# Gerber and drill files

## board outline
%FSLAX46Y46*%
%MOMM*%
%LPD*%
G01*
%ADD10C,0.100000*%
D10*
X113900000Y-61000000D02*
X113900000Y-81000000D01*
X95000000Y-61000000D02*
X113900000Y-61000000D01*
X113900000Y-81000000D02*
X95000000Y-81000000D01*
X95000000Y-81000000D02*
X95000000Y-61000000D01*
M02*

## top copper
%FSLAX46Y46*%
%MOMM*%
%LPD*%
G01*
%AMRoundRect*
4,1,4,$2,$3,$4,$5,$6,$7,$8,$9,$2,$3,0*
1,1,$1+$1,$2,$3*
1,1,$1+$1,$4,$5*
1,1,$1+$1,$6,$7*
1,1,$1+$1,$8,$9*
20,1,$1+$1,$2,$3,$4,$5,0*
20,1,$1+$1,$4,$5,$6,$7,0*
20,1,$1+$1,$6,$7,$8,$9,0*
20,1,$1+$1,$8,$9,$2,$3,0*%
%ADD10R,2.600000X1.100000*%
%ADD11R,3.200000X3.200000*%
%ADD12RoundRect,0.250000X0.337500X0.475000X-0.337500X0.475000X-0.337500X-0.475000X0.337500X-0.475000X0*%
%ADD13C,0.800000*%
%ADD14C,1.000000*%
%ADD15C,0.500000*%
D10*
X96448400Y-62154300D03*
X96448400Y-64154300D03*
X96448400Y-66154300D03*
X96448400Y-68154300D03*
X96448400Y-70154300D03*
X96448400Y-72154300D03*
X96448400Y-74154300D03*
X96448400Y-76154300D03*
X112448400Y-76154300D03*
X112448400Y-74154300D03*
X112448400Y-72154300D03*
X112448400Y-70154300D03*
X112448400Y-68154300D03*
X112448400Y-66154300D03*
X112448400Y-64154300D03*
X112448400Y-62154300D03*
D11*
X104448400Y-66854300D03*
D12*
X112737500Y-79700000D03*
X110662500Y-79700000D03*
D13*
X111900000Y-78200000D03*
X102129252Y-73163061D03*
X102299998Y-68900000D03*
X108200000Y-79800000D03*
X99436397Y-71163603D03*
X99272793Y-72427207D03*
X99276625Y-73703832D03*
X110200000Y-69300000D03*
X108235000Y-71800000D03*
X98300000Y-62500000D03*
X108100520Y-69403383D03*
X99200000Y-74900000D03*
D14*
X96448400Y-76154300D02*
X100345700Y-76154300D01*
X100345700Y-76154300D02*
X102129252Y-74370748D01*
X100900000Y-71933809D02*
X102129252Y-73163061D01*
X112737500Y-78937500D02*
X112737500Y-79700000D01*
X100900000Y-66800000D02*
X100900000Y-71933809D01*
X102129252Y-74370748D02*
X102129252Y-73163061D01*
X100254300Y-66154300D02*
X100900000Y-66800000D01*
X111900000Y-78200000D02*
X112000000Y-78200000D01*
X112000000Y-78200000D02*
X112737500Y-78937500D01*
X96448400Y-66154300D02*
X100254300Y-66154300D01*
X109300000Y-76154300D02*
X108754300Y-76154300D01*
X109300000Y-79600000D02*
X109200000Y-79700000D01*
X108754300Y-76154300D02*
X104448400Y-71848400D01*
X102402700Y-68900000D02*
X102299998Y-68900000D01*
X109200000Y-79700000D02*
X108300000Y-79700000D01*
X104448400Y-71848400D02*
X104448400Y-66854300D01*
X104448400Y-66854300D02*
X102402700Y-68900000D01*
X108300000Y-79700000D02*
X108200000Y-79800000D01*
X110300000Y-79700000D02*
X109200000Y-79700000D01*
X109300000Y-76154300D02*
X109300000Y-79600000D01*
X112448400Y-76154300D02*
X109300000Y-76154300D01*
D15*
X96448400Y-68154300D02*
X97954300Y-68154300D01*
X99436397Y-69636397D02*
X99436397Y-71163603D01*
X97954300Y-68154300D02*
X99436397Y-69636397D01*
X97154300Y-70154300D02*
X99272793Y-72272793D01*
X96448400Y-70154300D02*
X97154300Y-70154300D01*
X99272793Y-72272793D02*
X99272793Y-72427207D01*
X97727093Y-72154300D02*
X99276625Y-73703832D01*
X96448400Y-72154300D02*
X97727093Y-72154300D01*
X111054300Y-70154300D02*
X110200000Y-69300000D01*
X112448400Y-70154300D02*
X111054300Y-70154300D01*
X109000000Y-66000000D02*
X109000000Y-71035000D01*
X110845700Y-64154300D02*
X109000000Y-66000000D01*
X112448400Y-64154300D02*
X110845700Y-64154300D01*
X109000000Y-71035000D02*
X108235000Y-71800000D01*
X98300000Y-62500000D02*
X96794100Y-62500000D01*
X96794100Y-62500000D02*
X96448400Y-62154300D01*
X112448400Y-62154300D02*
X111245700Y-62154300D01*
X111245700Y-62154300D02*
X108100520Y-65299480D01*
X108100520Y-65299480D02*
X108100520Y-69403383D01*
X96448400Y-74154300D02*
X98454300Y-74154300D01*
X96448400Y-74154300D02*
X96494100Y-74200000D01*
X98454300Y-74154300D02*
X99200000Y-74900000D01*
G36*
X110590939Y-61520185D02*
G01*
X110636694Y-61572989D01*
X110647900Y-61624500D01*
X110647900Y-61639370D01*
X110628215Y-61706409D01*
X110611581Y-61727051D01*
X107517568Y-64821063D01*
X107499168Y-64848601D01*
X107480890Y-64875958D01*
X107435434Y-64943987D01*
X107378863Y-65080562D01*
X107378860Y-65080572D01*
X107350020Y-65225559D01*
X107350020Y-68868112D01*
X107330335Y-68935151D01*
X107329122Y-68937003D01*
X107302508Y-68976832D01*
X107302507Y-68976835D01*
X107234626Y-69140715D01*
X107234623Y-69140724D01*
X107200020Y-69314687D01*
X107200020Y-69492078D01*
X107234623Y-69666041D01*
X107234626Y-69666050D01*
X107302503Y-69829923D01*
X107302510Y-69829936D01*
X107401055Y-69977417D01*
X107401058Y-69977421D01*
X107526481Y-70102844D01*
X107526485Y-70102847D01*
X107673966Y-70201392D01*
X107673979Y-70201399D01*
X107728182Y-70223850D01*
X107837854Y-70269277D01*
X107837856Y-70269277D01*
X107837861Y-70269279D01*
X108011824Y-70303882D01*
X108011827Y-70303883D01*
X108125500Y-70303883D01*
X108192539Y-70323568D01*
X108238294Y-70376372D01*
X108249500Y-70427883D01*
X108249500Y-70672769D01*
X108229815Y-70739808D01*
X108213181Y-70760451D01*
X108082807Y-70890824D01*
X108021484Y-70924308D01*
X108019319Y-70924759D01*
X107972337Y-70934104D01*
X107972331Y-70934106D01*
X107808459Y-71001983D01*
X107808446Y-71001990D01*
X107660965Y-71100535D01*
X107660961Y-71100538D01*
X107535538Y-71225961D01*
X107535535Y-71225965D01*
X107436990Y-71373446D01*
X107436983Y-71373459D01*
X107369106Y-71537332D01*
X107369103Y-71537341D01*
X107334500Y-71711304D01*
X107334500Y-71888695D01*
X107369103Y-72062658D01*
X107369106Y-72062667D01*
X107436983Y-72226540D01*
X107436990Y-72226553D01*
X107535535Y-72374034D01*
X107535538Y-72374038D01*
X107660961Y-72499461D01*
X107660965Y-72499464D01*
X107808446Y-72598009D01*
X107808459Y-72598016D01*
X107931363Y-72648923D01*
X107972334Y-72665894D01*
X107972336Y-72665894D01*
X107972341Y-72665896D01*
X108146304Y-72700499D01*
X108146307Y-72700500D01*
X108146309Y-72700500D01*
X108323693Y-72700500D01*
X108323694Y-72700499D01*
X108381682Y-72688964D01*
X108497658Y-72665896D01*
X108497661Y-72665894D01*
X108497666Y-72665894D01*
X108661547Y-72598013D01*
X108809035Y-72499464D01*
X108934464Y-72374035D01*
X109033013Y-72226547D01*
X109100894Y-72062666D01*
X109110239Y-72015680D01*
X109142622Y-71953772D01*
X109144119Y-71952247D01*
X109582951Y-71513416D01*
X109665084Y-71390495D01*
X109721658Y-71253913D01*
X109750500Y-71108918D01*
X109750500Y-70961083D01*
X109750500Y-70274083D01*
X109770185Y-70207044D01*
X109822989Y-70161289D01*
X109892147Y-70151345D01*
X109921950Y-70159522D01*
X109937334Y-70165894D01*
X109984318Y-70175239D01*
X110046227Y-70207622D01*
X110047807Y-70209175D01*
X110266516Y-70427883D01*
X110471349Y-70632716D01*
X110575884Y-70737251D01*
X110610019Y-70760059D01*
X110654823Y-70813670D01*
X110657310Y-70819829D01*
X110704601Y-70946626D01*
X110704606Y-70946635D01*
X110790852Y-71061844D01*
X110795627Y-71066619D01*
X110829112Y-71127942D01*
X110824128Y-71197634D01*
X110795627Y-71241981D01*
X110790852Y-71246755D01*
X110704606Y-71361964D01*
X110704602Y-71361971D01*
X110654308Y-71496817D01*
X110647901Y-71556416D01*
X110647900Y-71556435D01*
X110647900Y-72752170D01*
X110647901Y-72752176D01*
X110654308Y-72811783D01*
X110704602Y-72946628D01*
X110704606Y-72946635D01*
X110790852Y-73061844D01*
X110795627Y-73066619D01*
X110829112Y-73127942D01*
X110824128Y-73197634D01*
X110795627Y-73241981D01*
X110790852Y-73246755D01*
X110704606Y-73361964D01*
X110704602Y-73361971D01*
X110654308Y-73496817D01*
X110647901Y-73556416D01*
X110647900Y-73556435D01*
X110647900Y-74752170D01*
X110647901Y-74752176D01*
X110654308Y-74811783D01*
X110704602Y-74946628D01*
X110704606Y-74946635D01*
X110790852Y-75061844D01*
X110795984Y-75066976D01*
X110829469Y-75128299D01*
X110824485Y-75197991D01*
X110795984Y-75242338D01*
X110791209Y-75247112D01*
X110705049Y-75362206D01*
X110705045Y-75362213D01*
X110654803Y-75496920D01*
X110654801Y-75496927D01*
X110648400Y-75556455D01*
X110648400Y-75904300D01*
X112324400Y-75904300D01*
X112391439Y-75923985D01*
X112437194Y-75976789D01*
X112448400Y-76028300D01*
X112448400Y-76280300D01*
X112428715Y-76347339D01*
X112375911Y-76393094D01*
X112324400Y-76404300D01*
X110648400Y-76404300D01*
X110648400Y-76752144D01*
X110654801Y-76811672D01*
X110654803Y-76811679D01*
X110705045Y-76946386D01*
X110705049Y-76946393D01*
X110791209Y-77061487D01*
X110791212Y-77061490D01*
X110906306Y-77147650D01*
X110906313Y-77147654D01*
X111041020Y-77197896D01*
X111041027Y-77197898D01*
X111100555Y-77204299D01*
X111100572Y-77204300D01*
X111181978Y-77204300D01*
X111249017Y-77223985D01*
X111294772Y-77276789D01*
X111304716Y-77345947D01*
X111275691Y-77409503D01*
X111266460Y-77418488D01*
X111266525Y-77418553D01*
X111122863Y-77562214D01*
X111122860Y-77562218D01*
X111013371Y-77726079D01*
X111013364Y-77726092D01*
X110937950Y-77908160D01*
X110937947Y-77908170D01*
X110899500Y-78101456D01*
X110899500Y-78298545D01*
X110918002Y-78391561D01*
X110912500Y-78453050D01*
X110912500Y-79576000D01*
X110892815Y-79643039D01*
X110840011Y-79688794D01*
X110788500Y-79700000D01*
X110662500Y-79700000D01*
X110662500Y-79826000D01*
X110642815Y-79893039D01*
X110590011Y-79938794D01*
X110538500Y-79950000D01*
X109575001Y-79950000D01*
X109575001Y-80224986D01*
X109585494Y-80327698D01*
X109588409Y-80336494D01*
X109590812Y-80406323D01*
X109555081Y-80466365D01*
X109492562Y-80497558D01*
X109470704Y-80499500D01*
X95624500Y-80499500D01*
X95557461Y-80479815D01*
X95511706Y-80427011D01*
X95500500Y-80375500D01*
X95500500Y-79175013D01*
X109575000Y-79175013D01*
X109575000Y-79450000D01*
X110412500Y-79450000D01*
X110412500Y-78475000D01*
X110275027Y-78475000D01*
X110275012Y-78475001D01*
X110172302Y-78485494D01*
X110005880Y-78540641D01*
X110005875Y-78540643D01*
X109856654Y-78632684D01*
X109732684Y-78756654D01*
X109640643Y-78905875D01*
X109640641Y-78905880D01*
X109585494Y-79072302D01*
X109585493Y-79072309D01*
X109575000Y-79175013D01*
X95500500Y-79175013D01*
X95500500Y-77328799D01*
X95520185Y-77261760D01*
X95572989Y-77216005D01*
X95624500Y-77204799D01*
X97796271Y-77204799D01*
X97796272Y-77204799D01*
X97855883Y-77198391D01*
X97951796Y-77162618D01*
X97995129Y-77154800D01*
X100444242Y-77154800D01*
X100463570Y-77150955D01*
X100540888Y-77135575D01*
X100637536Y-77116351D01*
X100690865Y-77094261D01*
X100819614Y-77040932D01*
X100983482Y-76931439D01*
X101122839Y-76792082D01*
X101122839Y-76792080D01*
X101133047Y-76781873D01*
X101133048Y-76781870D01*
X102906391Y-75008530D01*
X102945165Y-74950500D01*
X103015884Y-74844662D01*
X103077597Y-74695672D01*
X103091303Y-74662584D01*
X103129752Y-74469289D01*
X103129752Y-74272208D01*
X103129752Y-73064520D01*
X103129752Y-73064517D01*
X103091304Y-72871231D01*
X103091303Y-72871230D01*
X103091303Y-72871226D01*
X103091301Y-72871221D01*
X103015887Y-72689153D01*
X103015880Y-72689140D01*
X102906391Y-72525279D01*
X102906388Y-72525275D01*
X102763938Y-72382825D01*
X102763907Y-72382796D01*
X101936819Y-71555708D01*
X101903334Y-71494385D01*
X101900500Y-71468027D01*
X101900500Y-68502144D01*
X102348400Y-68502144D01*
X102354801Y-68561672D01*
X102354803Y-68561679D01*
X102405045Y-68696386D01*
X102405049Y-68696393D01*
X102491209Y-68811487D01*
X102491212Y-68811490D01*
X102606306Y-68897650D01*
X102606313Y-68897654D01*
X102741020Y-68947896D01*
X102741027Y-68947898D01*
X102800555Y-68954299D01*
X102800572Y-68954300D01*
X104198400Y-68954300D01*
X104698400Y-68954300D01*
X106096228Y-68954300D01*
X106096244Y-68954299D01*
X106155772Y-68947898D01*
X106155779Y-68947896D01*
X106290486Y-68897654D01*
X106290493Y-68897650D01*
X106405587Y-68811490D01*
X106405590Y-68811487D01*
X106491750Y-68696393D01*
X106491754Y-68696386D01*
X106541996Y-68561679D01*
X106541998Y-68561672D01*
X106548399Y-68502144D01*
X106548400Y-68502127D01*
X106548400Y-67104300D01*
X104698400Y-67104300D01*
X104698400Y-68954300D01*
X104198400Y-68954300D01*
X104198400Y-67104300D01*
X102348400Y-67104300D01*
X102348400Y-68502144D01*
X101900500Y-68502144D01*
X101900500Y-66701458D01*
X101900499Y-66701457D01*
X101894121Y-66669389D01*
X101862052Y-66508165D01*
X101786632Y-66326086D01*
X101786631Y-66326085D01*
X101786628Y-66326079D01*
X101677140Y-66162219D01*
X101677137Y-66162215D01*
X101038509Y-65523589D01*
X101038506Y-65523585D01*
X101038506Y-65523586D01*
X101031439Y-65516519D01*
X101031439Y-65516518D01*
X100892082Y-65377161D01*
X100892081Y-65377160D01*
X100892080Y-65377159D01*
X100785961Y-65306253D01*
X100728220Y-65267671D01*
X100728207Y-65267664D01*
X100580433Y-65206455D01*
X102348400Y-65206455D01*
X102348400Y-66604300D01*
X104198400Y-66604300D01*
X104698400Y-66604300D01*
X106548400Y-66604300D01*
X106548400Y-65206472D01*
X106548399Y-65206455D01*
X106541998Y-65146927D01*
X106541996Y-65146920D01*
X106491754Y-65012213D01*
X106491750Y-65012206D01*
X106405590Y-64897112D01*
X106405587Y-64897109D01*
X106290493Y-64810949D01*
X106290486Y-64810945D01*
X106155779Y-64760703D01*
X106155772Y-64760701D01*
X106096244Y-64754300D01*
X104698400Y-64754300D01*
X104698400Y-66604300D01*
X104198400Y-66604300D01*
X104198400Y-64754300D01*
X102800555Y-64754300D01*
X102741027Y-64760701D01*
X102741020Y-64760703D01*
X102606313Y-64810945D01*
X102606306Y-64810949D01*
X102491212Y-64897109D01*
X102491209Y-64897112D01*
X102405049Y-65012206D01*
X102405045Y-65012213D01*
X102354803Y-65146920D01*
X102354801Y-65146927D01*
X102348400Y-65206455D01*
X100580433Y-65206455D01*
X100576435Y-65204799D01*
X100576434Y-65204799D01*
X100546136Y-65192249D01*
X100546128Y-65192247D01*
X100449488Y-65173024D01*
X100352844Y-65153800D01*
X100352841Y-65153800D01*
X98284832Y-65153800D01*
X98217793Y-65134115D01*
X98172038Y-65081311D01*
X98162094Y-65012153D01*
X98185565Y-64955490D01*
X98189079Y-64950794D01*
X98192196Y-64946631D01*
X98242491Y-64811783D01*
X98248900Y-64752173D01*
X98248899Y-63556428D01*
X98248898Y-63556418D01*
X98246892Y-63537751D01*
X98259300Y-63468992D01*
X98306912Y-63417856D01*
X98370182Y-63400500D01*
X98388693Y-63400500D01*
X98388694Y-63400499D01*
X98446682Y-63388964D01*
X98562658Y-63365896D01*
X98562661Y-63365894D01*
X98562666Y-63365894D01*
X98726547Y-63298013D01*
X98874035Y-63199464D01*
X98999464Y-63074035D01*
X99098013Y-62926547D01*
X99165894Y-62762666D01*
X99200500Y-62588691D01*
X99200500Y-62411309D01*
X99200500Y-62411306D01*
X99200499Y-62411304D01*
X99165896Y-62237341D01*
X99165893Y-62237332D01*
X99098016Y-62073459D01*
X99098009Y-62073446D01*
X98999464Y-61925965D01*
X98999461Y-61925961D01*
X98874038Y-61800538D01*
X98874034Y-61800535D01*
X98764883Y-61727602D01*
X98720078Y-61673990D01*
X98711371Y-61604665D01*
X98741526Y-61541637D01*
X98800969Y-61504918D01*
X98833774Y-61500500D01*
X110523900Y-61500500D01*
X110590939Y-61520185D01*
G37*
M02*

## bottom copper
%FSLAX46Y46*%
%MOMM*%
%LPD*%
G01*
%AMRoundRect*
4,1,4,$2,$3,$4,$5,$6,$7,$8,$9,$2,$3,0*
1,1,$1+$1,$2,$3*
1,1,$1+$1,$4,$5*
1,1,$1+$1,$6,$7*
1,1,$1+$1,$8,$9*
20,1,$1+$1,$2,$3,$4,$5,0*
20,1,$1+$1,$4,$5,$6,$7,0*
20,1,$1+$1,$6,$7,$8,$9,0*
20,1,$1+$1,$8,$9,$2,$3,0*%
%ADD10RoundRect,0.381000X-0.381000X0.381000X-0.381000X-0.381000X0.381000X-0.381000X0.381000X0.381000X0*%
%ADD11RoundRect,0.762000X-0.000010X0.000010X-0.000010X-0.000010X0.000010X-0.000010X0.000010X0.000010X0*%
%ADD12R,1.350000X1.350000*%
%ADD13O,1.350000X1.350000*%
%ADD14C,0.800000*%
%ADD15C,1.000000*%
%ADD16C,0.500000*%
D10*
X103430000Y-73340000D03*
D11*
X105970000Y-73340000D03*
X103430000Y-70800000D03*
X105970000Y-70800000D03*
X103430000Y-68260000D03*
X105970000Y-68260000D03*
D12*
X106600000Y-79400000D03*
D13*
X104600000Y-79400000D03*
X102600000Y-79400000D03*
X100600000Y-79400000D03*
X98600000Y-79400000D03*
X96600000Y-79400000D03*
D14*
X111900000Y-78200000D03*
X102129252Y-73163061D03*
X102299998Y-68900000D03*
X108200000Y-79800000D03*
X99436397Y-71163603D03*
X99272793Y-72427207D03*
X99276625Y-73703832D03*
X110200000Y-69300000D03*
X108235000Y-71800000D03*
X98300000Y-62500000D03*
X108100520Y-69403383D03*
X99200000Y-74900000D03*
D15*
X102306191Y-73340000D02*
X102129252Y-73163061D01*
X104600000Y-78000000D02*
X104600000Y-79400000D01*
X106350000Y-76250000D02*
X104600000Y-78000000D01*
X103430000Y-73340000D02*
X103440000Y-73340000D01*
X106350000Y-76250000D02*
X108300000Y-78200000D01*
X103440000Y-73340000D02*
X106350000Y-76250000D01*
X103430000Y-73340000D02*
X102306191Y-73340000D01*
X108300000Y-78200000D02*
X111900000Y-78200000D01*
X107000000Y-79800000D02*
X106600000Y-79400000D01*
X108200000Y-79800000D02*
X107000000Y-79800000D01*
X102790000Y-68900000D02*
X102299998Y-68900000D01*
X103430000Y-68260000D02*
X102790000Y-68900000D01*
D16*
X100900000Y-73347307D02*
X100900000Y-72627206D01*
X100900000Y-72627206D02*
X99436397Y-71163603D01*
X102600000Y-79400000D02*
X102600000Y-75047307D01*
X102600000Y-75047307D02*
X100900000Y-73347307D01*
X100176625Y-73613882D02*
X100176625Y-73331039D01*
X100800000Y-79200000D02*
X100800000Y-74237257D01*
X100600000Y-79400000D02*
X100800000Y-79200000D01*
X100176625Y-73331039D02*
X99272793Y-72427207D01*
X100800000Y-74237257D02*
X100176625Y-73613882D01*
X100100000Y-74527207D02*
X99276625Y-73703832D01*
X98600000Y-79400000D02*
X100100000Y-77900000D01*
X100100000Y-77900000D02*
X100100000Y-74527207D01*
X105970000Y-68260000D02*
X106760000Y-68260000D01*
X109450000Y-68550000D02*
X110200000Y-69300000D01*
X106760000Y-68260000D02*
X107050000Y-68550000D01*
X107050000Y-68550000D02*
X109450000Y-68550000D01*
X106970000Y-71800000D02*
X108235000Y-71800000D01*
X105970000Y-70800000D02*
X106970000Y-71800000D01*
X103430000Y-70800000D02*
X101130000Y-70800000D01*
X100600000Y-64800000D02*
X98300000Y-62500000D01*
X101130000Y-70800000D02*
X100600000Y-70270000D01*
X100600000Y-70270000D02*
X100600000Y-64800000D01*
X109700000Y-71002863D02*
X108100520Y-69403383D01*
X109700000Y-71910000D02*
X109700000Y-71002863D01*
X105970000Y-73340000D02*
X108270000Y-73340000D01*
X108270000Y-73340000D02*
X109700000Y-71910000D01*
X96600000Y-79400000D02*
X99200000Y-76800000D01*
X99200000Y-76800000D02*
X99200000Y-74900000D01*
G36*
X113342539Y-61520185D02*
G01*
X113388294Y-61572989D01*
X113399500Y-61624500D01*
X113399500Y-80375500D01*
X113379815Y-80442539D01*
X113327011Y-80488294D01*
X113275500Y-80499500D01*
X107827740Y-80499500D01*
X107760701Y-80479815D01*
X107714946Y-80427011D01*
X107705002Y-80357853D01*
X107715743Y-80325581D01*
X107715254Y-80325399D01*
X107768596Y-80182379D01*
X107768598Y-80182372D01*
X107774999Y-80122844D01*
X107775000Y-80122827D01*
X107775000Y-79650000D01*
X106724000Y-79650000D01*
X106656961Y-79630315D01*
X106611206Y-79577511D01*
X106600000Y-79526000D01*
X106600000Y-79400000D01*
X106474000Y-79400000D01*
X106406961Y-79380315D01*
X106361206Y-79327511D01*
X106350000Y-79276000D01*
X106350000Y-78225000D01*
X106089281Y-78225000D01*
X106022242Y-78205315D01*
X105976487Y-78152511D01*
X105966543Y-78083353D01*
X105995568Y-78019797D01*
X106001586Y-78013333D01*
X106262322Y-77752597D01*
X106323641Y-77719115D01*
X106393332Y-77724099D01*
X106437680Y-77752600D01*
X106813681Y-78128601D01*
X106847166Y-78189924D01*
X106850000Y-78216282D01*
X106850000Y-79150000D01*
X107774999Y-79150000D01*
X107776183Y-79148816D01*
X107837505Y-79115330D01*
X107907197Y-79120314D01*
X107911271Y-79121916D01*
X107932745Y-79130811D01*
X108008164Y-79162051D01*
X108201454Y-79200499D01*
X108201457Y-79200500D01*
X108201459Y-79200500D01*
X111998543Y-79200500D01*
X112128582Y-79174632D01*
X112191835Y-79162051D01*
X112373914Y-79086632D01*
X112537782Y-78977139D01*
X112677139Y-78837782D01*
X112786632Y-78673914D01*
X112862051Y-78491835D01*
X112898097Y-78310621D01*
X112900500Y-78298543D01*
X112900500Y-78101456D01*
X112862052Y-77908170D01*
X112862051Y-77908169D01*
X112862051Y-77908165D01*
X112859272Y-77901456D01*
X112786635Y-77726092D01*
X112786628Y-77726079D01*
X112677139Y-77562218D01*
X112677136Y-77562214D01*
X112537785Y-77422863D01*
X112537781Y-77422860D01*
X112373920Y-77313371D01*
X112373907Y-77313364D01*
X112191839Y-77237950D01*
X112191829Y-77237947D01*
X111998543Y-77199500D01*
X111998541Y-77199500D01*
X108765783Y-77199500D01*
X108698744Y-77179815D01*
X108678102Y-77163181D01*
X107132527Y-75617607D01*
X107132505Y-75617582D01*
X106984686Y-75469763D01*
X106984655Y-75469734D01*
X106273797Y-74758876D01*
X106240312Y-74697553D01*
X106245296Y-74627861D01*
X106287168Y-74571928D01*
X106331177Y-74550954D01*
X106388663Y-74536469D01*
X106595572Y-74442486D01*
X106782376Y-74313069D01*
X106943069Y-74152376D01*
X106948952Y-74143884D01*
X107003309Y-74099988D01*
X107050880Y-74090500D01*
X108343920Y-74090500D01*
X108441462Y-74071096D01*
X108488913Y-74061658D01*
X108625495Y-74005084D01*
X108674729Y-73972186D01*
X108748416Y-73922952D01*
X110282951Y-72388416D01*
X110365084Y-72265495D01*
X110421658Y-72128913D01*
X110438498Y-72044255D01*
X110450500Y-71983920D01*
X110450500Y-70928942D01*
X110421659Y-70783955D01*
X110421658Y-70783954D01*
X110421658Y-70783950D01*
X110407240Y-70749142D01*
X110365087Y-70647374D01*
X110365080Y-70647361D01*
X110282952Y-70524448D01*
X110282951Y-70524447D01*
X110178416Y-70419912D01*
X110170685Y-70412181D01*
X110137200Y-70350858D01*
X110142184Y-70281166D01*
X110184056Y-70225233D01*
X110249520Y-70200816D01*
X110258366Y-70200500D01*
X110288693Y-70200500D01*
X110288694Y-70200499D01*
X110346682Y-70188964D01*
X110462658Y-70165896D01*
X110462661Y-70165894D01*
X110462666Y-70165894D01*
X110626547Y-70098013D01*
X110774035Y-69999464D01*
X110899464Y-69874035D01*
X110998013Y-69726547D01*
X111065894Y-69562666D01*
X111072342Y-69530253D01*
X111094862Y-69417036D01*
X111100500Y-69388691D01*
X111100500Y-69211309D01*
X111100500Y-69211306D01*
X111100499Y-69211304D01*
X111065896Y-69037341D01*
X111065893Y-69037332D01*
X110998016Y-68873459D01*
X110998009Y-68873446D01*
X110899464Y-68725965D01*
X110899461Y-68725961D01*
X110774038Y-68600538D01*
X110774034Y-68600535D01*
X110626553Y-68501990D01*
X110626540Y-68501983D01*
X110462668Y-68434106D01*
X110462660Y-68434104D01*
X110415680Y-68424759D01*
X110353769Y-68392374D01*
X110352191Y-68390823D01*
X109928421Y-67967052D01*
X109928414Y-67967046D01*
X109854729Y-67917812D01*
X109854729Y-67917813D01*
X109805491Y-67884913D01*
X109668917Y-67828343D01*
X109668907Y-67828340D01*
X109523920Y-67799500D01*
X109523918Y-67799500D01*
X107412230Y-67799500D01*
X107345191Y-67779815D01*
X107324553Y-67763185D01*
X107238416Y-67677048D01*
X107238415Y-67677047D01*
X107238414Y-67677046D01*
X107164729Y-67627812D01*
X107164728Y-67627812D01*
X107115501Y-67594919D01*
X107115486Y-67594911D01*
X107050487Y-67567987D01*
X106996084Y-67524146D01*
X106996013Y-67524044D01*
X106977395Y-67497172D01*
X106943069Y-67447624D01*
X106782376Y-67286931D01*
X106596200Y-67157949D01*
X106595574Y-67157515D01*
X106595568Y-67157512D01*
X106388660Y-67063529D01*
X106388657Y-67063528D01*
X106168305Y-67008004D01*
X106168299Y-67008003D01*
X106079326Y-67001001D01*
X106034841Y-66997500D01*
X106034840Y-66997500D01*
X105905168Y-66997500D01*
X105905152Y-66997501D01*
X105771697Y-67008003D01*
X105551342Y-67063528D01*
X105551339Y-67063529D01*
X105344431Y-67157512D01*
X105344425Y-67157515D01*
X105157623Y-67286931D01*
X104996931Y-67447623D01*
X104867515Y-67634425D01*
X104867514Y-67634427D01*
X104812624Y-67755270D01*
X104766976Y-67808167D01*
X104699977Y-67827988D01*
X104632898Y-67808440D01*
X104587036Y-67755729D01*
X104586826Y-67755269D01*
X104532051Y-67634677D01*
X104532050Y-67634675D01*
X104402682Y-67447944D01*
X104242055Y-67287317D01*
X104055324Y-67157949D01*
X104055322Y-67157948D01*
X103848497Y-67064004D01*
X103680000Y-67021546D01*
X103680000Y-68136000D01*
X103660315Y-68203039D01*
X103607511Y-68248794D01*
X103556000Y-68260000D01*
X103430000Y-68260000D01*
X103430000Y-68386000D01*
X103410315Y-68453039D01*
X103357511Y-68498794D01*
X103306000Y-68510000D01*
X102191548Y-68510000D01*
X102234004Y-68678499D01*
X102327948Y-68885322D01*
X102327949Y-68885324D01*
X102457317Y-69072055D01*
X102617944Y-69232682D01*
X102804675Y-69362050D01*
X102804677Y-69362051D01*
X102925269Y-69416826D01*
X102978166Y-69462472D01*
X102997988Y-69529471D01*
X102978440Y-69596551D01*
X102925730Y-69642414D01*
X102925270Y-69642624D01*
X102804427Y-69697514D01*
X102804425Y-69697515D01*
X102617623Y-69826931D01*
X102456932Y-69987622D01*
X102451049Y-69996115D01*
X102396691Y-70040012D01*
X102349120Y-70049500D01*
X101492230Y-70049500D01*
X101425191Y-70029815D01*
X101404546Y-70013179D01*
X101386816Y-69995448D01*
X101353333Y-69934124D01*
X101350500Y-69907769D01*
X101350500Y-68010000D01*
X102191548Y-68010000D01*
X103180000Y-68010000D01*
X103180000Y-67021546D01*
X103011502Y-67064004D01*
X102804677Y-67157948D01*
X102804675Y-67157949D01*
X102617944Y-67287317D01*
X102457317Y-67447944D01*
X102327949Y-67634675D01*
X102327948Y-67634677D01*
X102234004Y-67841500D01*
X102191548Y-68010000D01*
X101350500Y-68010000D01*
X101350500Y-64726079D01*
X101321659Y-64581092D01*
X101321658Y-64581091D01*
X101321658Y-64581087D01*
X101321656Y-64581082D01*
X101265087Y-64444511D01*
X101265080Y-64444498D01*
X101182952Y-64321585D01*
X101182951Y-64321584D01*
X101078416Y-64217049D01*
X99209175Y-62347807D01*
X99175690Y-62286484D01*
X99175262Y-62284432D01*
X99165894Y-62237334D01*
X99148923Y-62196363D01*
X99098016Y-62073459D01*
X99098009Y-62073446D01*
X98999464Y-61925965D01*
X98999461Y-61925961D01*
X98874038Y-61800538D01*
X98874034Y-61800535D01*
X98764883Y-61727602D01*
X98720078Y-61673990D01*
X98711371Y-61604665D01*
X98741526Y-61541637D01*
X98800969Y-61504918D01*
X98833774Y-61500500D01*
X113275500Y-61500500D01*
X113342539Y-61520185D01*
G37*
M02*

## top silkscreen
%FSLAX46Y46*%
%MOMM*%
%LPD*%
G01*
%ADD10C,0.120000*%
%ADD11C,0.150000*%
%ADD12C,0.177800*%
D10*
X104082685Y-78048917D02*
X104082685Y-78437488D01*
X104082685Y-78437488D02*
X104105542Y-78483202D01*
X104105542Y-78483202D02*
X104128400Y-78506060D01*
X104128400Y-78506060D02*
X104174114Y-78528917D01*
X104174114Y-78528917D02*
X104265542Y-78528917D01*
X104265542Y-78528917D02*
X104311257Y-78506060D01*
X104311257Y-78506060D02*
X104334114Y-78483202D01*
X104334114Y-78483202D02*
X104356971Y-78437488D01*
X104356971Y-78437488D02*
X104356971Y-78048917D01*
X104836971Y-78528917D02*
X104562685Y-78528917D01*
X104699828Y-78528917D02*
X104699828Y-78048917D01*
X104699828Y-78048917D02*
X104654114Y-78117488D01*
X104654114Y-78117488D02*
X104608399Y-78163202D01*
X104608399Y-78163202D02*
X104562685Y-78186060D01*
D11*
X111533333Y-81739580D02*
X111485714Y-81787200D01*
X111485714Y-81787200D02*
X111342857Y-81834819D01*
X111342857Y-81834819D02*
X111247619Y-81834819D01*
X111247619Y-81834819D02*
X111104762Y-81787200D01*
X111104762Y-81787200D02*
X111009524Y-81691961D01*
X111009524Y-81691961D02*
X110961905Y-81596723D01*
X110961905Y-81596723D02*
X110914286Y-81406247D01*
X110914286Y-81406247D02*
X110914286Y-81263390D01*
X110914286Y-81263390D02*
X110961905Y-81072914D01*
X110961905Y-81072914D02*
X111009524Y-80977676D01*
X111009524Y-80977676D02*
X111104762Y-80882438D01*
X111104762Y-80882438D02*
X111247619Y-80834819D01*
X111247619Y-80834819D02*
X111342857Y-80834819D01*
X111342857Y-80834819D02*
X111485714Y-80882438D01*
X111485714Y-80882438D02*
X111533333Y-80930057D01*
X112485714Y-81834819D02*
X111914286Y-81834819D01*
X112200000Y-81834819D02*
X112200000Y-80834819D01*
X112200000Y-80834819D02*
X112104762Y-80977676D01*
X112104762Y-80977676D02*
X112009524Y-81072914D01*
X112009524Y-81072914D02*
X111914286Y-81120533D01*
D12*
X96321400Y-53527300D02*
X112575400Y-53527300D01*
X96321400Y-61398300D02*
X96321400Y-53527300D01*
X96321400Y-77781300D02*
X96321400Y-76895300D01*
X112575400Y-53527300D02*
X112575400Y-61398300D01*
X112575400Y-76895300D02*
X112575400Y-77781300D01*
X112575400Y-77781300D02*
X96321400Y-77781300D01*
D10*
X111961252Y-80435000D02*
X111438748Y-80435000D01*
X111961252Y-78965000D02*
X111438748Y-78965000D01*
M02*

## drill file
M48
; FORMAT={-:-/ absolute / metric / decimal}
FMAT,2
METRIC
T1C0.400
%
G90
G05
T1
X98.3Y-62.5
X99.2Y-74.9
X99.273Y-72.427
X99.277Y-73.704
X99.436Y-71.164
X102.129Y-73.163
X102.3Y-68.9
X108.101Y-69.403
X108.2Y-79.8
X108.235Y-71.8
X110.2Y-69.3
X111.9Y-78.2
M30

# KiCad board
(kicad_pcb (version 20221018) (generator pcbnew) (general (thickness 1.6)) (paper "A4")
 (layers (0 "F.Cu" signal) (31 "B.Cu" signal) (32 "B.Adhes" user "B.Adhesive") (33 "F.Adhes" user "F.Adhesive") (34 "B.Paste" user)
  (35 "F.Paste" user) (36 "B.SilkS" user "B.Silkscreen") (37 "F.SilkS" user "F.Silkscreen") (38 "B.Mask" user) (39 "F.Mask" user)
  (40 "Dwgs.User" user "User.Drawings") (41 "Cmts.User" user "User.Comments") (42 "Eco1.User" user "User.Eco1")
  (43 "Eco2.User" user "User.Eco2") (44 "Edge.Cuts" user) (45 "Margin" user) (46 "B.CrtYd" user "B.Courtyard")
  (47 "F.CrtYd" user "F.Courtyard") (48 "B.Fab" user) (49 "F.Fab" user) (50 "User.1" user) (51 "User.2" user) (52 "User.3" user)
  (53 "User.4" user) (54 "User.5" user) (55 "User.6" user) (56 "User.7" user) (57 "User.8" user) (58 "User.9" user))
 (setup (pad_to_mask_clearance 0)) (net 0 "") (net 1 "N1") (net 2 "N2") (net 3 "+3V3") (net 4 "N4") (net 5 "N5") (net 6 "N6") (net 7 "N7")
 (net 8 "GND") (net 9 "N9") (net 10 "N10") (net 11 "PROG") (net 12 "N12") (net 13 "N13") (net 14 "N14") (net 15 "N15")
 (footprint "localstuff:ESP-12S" (layer "F.Cu") (at 104.4484 65.6543)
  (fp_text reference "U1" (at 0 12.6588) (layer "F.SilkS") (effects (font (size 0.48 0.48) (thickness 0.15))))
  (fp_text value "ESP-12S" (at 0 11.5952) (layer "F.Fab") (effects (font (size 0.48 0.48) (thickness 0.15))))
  (fp_line (start -8.127 -12.127) (end 8.127 -12.127) (stroke (width 0.1778) (type solid)) (layer "F.SilkS"))
  (fp_line (start -8.127 -4.256) (end -8.127 -12.127) (stroke (width 0.1778) (type solid)) (layer "F.SilkS"))
  (fp_line (start -8.127 12.127) (end -8.127 11.241) (stroke (width 0.1778) (type solid)) (layer "F.SilkS"))
  (fp_line (start 8.127 -12.127) (end 8.127 -4.256) (stroke (width 0.1778) (type solid)) (layer "F.SilkS"))
  (fp_line (start 8.127 11.241) (end 8.127 12.127) (stroke (width 0.1778) (type solid)) (layer "F.SilkS"))
  (fp_line (start 8.127 12.127) (end -8.127 12.127) (stroke (width 0.1778) (type solid)) (layer "F.SilkS"))
  (pad "1" smd rect (at -8 -3.5) (size 2.6 1.1) (layers "F.Cu" "F.Paste" "F.Mask") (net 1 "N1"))
  (pad "2" smd rect (at -8 -1.5) (size 2.6 1.1) (layers "F.Cu" "F.Paste" "F.Mask") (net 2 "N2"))
  (pad "3" smd rect (at -8 0.5) (size 2.6 1.1) (layers "F.Cu" "F.Paste" "F.Mask") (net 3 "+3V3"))
  (pad "4" smd rect (at -8 2.5) (size 2.6 1.1) (layers "F.Cu" "F.Paste" "F.Mask") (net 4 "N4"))
  (pad "5" smd rect (at -8 4.5) (size 2.6 1.1) (layers "F.Cu" "F.Paste" "F.Mask") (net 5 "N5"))
  (pad "6" smd rect (at -8 6.5) (size 2.6 1.1) (layers "F.Cu" "F.Paste" "F.Mask") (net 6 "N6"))
  (pad "7" smd rect (at -8 8.5) (size 2.6 1.1) (layers "F.Cu" "F.Paste" "F.Mask") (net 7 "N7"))
  (pad "8" smd rect (at -8 10.5) (size 2.6 1.1) (layers "F.Cu" "F.Paste" "F.Mask") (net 3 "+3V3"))
  (pad "9" smd rect (at 8 10.5 180) (size 2.6 1.1) (layers "F.Cu" "F.Paste" "F.Mask") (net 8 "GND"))
  (pad "10" smd rect (at 8 8.5 180) (size 2.6 1.1) (layers "F.Cu" "F.Paste" "F.Mask") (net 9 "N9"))
  (pad "11" smd rect (at 8 6.5 180) (size 2.6 1.1) (layers "F.Cu" "F.Paste" "F.Mask") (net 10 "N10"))
  (pad "12" smd rect (at 8 4.5 180) (size 2.6 1.1) (layers "F.Cu" "F.Paste" "F.Mask") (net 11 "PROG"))
  (pad "13" smd rect (at 8 2.5 180) (size 2.6 1.1) (layers "F.Cu" "F.Paste" "F.Mask") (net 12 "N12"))
  (pad "14" smd rect (at 8 0.5 180) (size 2.6 1.1) (layers "F.Cu" "F.Paste" "F.Mask") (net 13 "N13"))
  (pad "15" smd rect (at 8 -1.5 180) (size 2.6 1.1) (layers "F.Cu" "F.Paste" "F.Mask") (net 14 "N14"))
  (pad "16" smd rect (at 8 -3.5 180) (size 2.6 1.1) (layers "F.Cu" "F.Paste" "F.Mask") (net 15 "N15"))
  (pad "P$1" smd rect (at 0 1.2) (size 3.2 3.2) (layers "F.Cu" "F.Mask") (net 8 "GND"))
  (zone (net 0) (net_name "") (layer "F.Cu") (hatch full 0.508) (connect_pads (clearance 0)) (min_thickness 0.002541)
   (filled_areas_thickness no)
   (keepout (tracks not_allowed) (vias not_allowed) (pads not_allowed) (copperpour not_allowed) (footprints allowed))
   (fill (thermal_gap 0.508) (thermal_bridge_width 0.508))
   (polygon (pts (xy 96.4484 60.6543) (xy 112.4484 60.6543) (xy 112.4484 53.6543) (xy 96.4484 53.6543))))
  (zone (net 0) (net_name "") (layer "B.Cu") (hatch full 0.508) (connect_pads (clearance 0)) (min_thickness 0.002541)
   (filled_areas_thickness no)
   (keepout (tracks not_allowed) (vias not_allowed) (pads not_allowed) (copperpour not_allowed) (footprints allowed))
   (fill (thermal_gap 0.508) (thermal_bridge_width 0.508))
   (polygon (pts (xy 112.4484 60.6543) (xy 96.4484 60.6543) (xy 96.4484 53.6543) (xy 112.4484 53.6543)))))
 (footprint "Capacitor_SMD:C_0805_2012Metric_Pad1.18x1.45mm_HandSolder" (layer "F.Cu") (at 111.7 79.7 180)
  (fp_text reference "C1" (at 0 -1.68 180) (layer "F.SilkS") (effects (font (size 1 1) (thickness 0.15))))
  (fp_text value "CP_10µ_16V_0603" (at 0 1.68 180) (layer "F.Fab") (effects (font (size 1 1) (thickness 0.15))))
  (fp_line (start -0.261252 -0.735) (end 0.261252 -0.735) (stroke (width 0.12) (type solid)) (layer "F.SilkS"))
  (fp_line (start -0.261252 0.735) (end 0.261252 0.735) (stroke (width 0.12) (type solid)) (layer "F.SilkS"))
  (pad "1" smd roundrect (at -1.0375 0 180) (size 1.175 1.45) (layers "F.Cu" "F.Paste" "F.Mask") (roundrect_rratio 0.2127659574)
   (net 3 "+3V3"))
  (pad "2" smd roundrect (at 1.0375 0 180) (size 1.175 1.45) (layers "F.Cu" "F.Paste" "F.Mask") (roundrect_rratio 0.2127659574)
   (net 8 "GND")))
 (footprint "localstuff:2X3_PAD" (layer "B.Cu") (at 104.7 70.8 90)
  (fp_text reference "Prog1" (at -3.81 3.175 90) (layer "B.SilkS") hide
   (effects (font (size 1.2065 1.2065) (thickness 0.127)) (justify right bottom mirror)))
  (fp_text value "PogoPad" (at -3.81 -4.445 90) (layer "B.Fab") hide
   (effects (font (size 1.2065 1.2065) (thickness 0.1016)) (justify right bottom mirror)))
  (pad "1" smd roundrect (at -2.54 -1.27 270) (size 1.524 1.524) (layers "B.Cu" "B.Paste" "B.Mask") (roundrect_rratio 0.25) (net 3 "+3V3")
   (solder_mask_margin 0.1016))
  (pad "2" smd roundrect (at -2.54 1.27 270) (size 1.524 1.524) (layers "B.Cu" "B.Paste" "B.Mask") (roundrect_rratio 0.5) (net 15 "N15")
   (solder_mask_margin 0.1016))
  (pad "3" smd roundrect (at 0 -1.27 270) (size 1.524 1.524) (layers "B.Cu" "B.Paste" "B.Mask") (roundrect_rratio 0.5) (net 1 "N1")
   (solder_mask_margin 0.1016))
  (pad "4" smd roundrect (at 0 1.27 270) (size 1.524 1.524) (layers "B.Cu" "B.Paste" "B.Mask") (roundrect_rratio 0.5) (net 14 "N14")
   (solder_mask_margin 0.1016))
  (pad "5" smd roundrect (at 2.54 -1.27 270) (size 1.524 1.524) (layers "B.Cu" "B.Paste" "B.Mask") (roundrect_rratio 0.5) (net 8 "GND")
   (solder_mask_margin 0.1016))
  (pad "6" smd roundrect (at 2.54 1.27 270) (size 1.524 1.524) (layers "B.Cu" "B.Paste" "B.Mask") (roundrect_rratio 0.5) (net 11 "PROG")
   (solder_mask_margin 0.1016)))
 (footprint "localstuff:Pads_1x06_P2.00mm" (layer "B.Cu") (at 106.6 79.4 90)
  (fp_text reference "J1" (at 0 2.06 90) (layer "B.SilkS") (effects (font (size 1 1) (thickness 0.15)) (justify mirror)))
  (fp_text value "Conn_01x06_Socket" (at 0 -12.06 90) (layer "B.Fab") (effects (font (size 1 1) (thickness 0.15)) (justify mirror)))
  (pad "1" smd rect (at 0 0 90) (size 1.35 1.35) (layers "B.Cu" "B.Paste" "B.Mask") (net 8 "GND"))
  (pad "2" smd oval (at 0 -2 90) (size 1.35 1.35) (layers "B.Cu" "B.Paste" "B.Mask") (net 3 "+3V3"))
  (pad "3" smd oval (at 0 -4 90) (size 1.35 1.35) (layers "B.Cu" "B.Paste" "B.Mask") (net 4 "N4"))
  (pad "4" smd oval (at 0 -6 90) (size 1.35 1.35) (layers "B.Cu" "B.Paste" "B.Mask") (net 5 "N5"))
  (pad "5" smd oval (at 0 -8 90) (size 1.35 1.35) (layers "B.Cu" "B.Paste" "B.Mask") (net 6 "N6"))
  (pad "6" smd oval (at 0 -10 90) (size 1.35 1.35) (layers "B.Cu" "B.Paste" "B.Mask") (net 7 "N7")))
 (gr_line (start 113.9 61) (end 113.9 81) (stroke (width 0.1) (type default)) (layer "Edge.Cuts"))
 (gr_line (start 95 61) (end 113.9 61) (stroke (width 0.1) (type default)) (layer "Edge.Cuts"))
 (gr_line (start 113.9 81) (end 95 81) (stroke (width 0.1) (type default)) (layer "Edge.Cuts"))
 (gr_line (start 95 81) (end 95 61) (stroke (width 0.1) (type default)) (layer "Edge.Cuts"))
 (segment (start 96.4484 76.1543) (end 100.3457 76.1543) (width 1) (layer "F.Cu") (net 3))
 (segment (start 100.3457 76.1543) (end 102.129252 74.370748) (width 1) (layer "F.Cu") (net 3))
 (segment (start 100.9 71.933809) (end 102.129252 73.163061) (width 1) (layer "F.Cu") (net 3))
 (segment (start 112.7375 78.9375) (end 112.7375 79.7) (width 1) (layer "F.Cu") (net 3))
 (segment (start 100.9 66.8) (end 100.9 71.933809) (width 1) (layer "F.Cu") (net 3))
 (segment (start 102.129252 74.370748) (end 102.129252 73.163061) (width 1) (layer "F.Cu") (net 3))
 (segment (start 100.2543 66.1543) (end 100.9 66.8) (width 1) (layer "F.Cu") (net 3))
 (segment (start 111.9 78.2) (end 112 78.2) (width 1) (layer "F.Cu") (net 3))
 (segment (start 112 78.2) (end 112.7375 78.9375) (width 1) (layer "F.Cu") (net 3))
 (segment (start 96.4484 66.1543) (end 100.2543 66.1543) (width 1) (layer "F.Cu") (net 3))
 (via (at 111.9 78.2) (size 0.8) (drill 0.4) (layers "F.Cu" "B.Cu") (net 3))
 (via (at 102.129252 73.163061) (size 0.8) (drill 0.4) (layers "F.Cu" "B.Cu") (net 3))
 (segment (start 102.306191 73.34) (end 102.129252 73.163061) (width 1) (layer "B.Cu") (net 3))
 (segment (start 104.6 78) (end 104.6 79.4) (width 1) (layer "B.Cu") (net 3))
 (segment (start 106.35 76.25) (end 104.6 78) (width 1) (layer "B.Cu") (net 3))
 (segment (start 103.43 73.34) (end 103.44 73.34) (width 1) (layer "B.Cu") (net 3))
 (segment (start 106.35 76.25) (end 108.3 78.2) (width 1) (layer "B.Cu") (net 3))
 (segment (start 103.44 73.34) (end 106.35 76.25) (width 1) (layer "B.Cu") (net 3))
 (segment (start 103.43 73.34) (end 102.306191 73.34) (width 1) (layer "B.Cu") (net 3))
 (segment (start 108.3 78.2) (end 111.9 78.2) (width 1) (layer "B.Cu") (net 3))
 (segment (start 109.3 76.1543) (end 108.7543 76.1543) (width 1) (layer "F.Cu") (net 8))
 (segment (start 109.3 79.6) (end 109.2 79.7) (width 1) (layer "F.Cu") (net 8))
 (segment (start 108.7543 76.1543) (end 104.4484 71.8484) (width 1) (layer "F.Cu") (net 8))
 (segment (start 102.4027 68.9) (end 102.299998 68.9) (width 1) (layer "F.Cu") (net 8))
 (segment (start 109.2 79.7) (end 108.3 79.7) (width 1) (layer "F.Cu") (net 8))
 (segment (start 104.4484 71.8484) (end 104.4484 66.8543) (width 1) (layer "F.Cu") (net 8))
 (segment (start 104.4484 66.8543) (end 102.4027 68.9) (width 1) (layer "F.Cu") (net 8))
 (segment (start 108.3 79.7) (end 108.2 79.8) (width 1) (layer "F.Cu") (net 8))
 (segment (start 110.3 79.7) (end 109.2 79.7) (width 1) (layer "F.Cu") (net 8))
 (segment (start 109.3 76.1543) (end 109.3 79.6) (width 1) (layer "F.Cu") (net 8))
 (segment (start 112.4484 76.1543) (end 109.3 76.1543) (width 1) (layer "F.Cu") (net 8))
 (via (at 102.299998 68.9) (size 0.8) (drill 0.4) (layers "F.Cu" "B.Cu") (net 8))
 (via (at 108.2 79.8) (size 0.8) (drill 0.4) (layers "F.Cu" "B.Cu") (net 8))
 (segment (start 107 79.8) (end 106.6 79.4) (width 1) (layer "B.Cu") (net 8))
 (segment (start 108.2 79.8) (end 107 79.8) (width 1) (layer "B.Cu") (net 8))
 (segment (start 102.79 68.9) (end 102.299998 68.9) (width 1) (layer "B.Cu") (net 8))
 (segment (start 103.43 68.26) (end 102.79 68.9) (width 1) (layer "B.Cu") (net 8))
 (segment (start 96.4484 68.1543) (end 97.9543 68.1543) (width 0.5) (layer "F.Cu") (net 4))
 (segment (start 99.436397 69.636397) (end 99.436397 71.163603) (width 0.5) (layer "F.Cu") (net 4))
 (segment (start 97.9543 68.1543) (end 99.436397 69.636397) (width 0.5) (layer "F.Cu") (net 4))
 (via (at 99.436397 71.163603) (size 0.8) (drill 0.4) (layers "F.Cu" "B.Cu") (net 4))
 (segment (start 100.9 73.347307) (end 100.9 72.627206) (width 0.5) (layer "B.Cu") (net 4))
 (segment (start 100.9 72.627206) (end 99.436397 71.163603) (width 0.5) (layer "B.Cu") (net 4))
 (segment (start 102.6 79.4) (end 102.6 75.047307) (width 0.5) (layer "B.Cu") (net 4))
 (segment (start 102.6 75.047307) (end 100.9 73.347307) (width 0.5) (layer "B.Cu") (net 4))
 (segment (start 97.1543 70.1543) (end 99.272793 72.272793) (width 0.5) (layer "F.Cu") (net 5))
 (segment (start 96.4484 70.1543) (end 97.1543 70.1543) (width 0.5) (layer "F.Cu") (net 5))
 (segment (start 99.272793 72.272793) (end 99.272793 72.427207) (width 0.5) (layer "F.Cu") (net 5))
 (via (at 99.272793 72.427207) (size 0.8) (drill 0.4) (layers "F.Cu" "B.Cu") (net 5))
 (segment (start 100.176625 73.613882) (end 100.176625 73.331039) (width 0.5) (layer "B.Cu") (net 5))
 (segment (start 100.8 79.2) (end 100.8 74.237257) (width 0.5) (layer "B.Cu") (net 5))
 (segment (start 100.6 79.4) (end 100.8 79.2) (width 0.5) (layer "B.Cu") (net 5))
 (segment (start 100.176625 73.331039) (end 99.272793 72.427207) (width 0.5) (layer "B.Cu") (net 5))
 (segment (start 100.8 74.237257) (end 100.176625 73.613882) (width 0.5) (layer "B.Cu") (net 5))
 (segment (start 97.727093 72.1543) (end 99.276625 73.703832) (width 0.5) (layer "F.Cu") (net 6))
 (segment (start 96.4484 72.1543) (end 97.727093 72.1543) (width 0.5) (layer "F.Cu") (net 6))
 (via (at 99.276625 73.703832) (size 0.8) (drill 0.4) (layers "F.Cu" "B.Cu") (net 6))
 (segment (start 100.1 74.527207) (end 99.276625 73.703832) (width 0.5) (layer "B.Cu") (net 6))
 (segment (start 98.6 79.4) (end 100.1 77.9) (width 0.5) (layer "B.Cu") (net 6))
 (segment (start 100.1 77.9) (end 100.1 74.527207) (width 0.5) (layer "B.Cu") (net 6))
 (segment (start 111.0543 70.1543) (end 110.2 69.3) (width 0.5) (layer "F.Cu") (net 11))
 (segment (start 112.4484 70.1543) (end 111.0543 70.1543) (width 0.5) (layer "F.Cu") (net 11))
 (via (at 110.2 69.3) (size 0.8) (drill 0.4) (layers "F.Cu" "B.Cu") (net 11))
 (segment (start 105.97 68.26) (end 106.76 68.26) (width 0.5) (layer "B.Cu") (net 11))
 (segment (start 109.45 68.55) (end 110.2 69.3) (width 0.5) (layer "B.Cu") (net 11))
 (segment (start 106.76 68.26) (end 107.05 68.55) (width 0.5) (layer "B.Cu") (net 11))
 (segment (start 107.05 68.55) (end 109.45 68.55) (width 0.5) (layer "B.Cu") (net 11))
 (segment (start 109 66) (end 109 71.035) (width 0.5) (layer "F.Cu") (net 14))
 (segment (start 110.8457 64.1543) (end 109 66) (width 0.5) (layer "F.Cu") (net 14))
 (segment (start 112.4484 64.1543) (end 110.8457 64.1543) (width 0.5) (layer "F.Cu") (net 14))
 (segment (start 109 71.035) (end 108.235 71.8) (width 0.5) (layer "F.Cu") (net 14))
 (via (at 108.235 71.8) (size 0.8) (drill 0.4) (layers "F.Cu" "B.Cu") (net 14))
 (segment (start 106.97 71.8) (end 108.235 71.8) (width 0.5) (layer "B.Cu") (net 14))
 (segment (start 105.97 70.8) (end 106.97 71.8) (width 0.5) (layer "B.Cu") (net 14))
 (segment (start 98.3 62.5) (end 96.7941 62.5) (width 0.5) (layer "F.Cu") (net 1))
 (segment (start 96.7941 62.5) (end 96.4484 62.1543) (width 0.5) (layer "F.Cu") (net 1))
 (via (at 98.3 62.5) (size 0.8) (drill 0.4) (layers "F.Cu" "B.Cu") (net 1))
 (segment (start 103.43 70.8) (end 101.13 70.8) (width 0.5) (layer "B.Cu") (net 1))
 (segment (start 100.6 64.8) (end 98.3 62.5) (width 0.5) (layer "B.Cu") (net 1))
 (segment (start 101.13 70.8) (end 100.6 70.27) (width 0.5) (layer "B.Cu") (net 1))
 (segment (start 100.6 70.27) (end 100.6 64.8) (width 0.5) (layer "B.Cu") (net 1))
 (segment (start 112.4484 62.1543) (end 111.2457 62.1543) (width 0.5) (layer "F.Cu") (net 15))
 (segment (start 111.2457 62.1543) (end 108.10052 65.29948) (width 0.5) (layer "F.Cu") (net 15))
 (segment (start 108.10052 65.29948) (end 108.10052 69.403383) (width 0.5) (layer "F.Cu") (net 15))
 (via (at 108.10052 69.403383) (size 0.8) (drill 0.4) (layers "F.Cu" "B.Cu") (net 15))
 (segment (start 109.7 71.002863) (end 108.10052 69.403383) (width 0.5) (layer "B.Cu") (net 15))
 (segment (start 109.7 71.91) (end 109.7 71.002863) (width 0.5) (layer "B.Cu") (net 15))
 (segment (start 105.97 73.34) (end 108.27 73.34) (width 0.5) (layer "B.Cu") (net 15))
 (segment (start 108.27 73.34) (end 109.7 71.91) (width 0.5) (layer "B.Cu") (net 15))
 (segment (start 96.4484 74.1543) (end 98.4543 74.1543) (width 0.5) (layer "F.Cu") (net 7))
 (segment (start 96.4484 74.1543) (end 96.4941 74.2) (width 0.5) (layer "F.Cu") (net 7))
 (segment (start 98.4543 74.1543) (end 99.2 74.9) (width 0.5) (layer "F.Cu") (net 7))
 (via (at 99.2 74.9) (size 0.8) (drill 0.4) (layers "F.Cu" "B.Cu") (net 7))
 (segment (start 96.6 79.4) (end 99.2 76.8) (width 0.5) (layer "B.Cu") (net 7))
 (segment (start 99.2 76.8) (end 99.2 74.9) (width 0.5) (layer "B.Cu") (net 7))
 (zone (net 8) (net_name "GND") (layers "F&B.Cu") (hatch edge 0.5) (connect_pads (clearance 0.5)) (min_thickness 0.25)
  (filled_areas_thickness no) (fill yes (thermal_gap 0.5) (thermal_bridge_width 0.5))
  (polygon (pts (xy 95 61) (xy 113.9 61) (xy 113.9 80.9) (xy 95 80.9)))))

